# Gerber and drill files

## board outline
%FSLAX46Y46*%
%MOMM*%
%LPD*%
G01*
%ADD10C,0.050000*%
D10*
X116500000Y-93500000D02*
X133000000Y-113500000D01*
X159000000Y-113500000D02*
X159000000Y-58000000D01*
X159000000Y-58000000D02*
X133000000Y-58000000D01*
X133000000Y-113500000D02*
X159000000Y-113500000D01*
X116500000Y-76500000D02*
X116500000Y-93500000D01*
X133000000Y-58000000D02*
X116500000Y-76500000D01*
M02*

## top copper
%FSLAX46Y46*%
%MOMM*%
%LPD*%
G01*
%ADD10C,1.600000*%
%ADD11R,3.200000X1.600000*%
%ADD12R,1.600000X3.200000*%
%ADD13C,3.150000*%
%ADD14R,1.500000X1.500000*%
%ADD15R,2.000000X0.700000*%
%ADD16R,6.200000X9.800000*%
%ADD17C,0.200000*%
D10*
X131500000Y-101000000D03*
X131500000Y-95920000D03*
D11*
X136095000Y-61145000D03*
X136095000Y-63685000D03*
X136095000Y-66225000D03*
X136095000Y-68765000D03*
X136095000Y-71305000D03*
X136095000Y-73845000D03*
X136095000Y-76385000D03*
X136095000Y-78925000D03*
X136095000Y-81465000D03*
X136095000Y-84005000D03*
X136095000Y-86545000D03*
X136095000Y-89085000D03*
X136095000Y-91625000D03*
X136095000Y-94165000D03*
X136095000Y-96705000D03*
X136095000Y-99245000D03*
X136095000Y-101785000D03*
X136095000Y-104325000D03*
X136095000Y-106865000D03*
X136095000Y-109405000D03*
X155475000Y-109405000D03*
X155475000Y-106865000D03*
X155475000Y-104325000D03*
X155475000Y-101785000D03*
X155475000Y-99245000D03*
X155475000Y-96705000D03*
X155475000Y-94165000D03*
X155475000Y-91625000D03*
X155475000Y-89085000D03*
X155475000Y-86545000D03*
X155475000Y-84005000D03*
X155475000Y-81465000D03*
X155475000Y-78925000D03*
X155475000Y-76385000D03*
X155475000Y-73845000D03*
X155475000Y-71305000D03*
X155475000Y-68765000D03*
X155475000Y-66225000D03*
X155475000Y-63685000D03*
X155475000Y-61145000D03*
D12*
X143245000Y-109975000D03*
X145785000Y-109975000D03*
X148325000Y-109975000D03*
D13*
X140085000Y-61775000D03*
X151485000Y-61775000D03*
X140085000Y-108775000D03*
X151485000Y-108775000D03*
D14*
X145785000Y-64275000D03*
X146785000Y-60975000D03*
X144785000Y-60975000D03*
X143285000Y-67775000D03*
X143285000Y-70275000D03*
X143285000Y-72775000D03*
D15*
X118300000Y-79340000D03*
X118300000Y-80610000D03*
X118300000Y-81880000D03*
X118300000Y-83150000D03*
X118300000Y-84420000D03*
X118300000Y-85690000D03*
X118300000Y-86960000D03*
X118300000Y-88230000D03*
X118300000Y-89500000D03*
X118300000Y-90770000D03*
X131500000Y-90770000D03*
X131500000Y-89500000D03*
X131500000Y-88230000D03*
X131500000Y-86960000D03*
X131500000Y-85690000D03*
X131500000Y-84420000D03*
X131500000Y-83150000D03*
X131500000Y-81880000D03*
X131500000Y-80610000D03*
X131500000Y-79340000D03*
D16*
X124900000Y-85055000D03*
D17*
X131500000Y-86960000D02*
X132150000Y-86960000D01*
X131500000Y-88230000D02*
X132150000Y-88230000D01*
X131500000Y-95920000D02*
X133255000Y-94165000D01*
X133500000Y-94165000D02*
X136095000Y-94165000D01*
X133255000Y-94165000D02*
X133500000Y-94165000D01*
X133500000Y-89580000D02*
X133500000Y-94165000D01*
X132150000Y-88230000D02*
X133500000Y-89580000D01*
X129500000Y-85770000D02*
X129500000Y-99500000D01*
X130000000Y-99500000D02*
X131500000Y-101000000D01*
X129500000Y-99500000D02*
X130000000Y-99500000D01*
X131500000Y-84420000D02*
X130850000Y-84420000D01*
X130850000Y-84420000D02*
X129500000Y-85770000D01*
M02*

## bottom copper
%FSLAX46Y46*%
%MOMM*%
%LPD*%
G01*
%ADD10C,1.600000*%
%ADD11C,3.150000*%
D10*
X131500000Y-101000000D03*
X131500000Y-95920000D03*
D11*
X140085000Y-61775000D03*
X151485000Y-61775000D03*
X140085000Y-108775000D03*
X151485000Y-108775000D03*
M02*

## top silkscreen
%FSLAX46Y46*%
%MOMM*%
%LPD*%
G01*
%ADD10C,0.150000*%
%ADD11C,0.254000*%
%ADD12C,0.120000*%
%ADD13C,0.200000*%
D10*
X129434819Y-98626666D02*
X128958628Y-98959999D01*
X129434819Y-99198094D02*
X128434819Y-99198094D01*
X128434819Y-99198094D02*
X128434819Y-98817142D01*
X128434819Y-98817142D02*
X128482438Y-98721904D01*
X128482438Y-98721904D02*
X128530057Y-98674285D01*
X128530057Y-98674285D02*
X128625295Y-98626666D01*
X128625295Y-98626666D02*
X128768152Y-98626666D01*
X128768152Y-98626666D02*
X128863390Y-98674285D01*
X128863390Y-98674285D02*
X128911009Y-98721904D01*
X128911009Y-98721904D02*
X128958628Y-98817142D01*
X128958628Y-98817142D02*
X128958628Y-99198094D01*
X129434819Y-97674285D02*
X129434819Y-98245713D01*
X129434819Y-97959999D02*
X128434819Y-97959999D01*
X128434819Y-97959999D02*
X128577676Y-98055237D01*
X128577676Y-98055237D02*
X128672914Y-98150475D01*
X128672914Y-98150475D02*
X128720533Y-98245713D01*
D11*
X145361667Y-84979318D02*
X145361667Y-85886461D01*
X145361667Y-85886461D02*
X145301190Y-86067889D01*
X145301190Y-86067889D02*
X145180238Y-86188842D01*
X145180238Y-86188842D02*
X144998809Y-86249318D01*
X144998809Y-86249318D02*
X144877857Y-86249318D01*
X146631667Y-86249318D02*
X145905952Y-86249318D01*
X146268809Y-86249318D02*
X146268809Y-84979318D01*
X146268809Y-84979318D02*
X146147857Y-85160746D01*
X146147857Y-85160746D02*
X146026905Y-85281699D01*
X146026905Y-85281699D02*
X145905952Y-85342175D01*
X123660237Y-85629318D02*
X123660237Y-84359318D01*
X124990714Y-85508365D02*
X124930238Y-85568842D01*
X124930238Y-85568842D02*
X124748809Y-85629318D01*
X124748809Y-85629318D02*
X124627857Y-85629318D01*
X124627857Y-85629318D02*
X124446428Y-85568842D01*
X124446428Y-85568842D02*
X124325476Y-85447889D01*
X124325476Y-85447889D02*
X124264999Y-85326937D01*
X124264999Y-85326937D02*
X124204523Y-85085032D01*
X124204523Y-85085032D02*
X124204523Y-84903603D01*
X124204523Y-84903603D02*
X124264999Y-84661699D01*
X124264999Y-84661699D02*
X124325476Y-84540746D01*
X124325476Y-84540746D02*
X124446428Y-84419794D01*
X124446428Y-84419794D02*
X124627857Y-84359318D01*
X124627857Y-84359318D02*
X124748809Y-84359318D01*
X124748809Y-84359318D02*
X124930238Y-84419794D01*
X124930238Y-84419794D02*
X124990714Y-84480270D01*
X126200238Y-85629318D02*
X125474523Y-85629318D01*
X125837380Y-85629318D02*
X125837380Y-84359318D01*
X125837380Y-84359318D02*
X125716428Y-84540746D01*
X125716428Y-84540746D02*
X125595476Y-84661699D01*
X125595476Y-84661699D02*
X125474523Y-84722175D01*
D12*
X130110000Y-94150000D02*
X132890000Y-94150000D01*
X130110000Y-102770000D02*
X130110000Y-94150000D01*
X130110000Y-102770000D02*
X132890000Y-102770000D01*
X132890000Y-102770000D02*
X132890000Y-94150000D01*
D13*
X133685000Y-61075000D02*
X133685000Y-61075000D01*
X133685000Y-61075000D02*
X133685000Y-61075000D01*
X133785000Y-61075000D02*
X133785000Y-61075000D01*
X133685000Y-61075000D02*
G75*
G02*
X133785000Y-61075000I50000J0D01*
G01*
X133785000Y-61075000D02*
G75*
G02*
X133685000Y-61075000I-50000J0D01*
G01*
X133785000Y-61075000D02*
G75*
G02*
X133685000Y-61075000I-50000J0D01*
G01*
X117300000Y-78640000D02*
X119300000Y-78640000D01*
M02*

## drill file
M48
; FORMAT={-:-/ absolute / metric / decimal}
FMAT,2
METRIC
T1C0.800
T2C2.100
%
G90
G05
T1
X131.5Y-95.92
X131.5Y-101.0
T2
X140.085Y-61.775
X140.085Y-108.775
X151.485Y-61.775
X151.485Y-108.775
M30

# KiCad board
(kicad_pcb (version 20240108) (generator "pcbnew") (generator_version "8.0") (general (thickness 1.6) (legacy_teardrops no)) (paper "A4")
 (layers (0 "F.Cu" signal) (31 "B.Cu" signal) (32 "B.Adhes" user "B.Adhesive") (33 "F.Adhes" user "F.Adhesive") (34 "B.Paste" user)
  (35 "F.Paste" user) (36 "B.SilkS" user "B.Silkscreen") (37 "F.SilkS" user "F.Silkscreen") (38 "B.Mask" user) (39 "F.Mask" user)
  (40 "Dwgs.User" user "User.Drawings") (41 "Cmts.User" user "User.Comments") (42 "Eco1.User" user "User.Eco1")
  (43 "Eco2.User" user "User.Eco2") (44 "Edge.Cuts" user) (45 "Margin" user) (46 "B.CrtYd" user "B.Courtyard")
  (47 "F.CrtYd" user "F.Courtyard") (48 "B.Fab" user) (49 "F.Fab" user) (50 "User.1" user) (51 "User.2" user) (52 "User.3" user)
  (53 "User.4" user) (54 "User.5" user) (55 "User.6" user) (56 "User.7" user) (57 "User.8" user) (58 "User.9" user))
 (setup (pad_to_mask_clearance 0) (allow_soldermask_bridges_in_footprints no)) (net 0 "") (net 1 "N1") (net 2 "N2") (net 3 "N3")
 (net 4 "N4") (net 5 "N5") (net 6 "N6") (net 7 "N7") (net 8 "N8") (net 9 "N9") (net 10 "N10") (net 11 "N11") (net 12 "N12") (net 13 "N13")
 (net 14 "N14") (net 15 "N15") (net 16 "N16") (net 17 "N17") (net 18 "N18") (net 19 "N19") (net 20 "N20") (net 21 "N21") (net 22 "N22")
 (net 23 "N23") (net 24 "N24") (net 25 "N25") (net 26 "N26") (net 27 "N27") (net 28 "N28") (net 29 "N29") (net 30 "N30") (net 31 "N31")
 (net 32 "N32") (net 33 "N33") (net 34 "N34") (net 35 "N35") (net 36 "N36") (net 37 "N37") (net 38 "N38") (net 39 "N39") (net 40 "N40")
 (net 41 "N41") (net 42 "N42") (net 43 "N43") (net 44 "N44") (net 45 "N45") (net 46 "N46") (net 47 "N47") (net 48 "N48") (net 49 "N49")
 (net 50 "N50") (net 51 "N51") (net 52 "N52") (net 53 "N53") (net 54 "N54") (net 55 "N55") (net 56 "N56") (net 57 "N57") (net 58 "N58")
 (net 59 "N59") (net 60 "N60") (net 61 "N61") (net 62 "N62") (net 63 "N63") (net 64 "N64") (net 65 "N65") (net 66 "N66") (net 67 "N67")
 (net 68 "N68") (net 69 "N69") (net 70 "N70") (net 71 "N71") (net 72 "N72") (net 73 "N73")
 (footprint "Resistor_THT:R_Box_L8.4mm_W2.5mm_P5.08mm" (layer "F.Cu") (at 131.5 101 90)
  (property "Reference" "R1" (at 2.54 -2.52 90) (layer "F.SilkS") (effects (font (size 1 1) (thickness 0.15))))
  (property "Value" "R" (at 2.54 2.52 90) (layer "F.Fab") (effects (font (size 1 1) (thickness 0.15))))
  (fp_line (start 6.85 -1.39) (end 6.85 1.39) (stroke (width 0.12) (type solid)) (layer "F.SilkS"))
  (fp_line (start -1.77 -1.39) (end 6.85 -1.39) (stroke (width 0.12) (type solid)) (layer "F.SilkS"))
  (fp_line (start -1.77 -1.39) (end -1.77 1.39) (stroke (width 0.12) (type solid)) (layer "F.SilkS"))
  (fp_line (start -1.77 1.39) (end 6.85 1.39) (stroke (width 0.12) (type solid)) (layer "F.SilkS"))
  (pad "1" thru_hole circle (at 0 0 90) (size 1.6 1.6) (drill 0.8) (layers "*.Cu" "*.Mask") (remove_unused_layers no) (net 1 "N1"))
  (pad "2" thru_hole circle (at 5.08 0 90) (size 1.6 1.6) (drill 0.8) (layers "*.Cu" "*.Mask") (remove_unused_layers no) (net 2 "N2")))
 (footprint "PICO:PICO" (layer "F.Cu") (at 145.785 85.275)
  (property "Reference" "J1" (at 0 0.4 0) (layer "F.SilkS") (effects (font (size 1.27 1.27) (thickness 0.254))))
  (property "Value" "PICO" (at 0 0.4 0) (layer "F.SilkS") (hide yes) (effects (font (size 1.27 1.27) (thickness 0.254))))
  (fp_line (start -12.1 -24.2) (end -12.1 -24.2) (stroke (width 0.2) (type solid)) (layer "F.SilkS"))
  (fp_line (start -12.1 -24.2) (end -12.1 -24.2) (stroke (width 0.2) (type solid)) (layer "F.SilkS"))
  (fp_line (start -12 -24.2) (end -12 -24.2) (stroke (width 0.2) (type solid)) (layer "F.SilkS"))
  (fp_arc (start -12.1 -24.2) (mid -12.05 -24.25) (end -12 -24.2) (stroke (width 0.2) (type solid)) (layer "F.SilkS"))
  (fp_arc (start -12 -24.2) (mid -12.05 -24.15) (end -12.1 -24.2) (stroke (width 0.2) (type solid)) (layer "F.SilkS"))
  (fp_arc (start -12 -24.2) (mid -12.05 -24.15) (end -12.1 -24.2) (stroke (width 0.2) (type solid)) (layer "F.SilkS"))
  (pad "1" smd rect (at -9.69 -24.13 90) (size 1.6 3.2) (layers "F.Cu" "F.Paste" "F.Mask") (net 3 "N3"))
  (pad "2" smd rect (at -9.69 -21.59 90) (size 1.6 3.2) (layers "F.Cu" "F.Paste" "F.Mask") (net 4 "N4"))
  (pad "3" smd rect (at -9.69 -19.05 90) (size 1.6 3.2) (layers "F.Cu" "F.Paste" "F.Mask") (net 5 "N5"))
  (pad "4" smd rect (at -9.69 -16.51 90) (size 1.6 3.2) (layers "F.Cu" "F.Paste" "F.Mask") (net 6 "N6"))
  (pad "5" smd rect (at -9.69 -13.97 90) (size 1.6 3.2) (layers "F.Cu" "F.Paste" "F.Mask") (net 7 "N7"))
  (pad "6" smd rect (at -9.69 -11.43 90) (size 1.6 3.2) (layers "F.Cu" "F.Paste" "F.Mask") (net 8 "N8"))
  (pad "7" smd rect (at -9.69 -8.89 90) (size 1.6 3.2) (layers "F.Cu" "F.Paste" "F.Mask") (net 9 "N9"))
  (pad "8" smd rect (at -9.69 -6.35 90) (size 1.6 3.2) (layers "F.Cu" "F.Paste" "F.Mask") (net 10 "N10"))
  (pad "9" smd rect (at -9.69 -3.81 90) (size 1.6 3.2) (layers "F.Cu" "F.Paste" "F.Mask") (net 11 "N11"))
  (pad "10" smd rect (at -9.69 -1.27 90) (size 1.6 3.2) (layers "F.Cu" "F.Paste" "F.Mask") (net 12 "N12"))
  (pad "11" smd rect (at -9.69 1.27 90) (size 1.6 3.2) (layers "F.Cu" "F.Paste" "F.Mask") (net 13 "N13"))
  (pad "12" smd rect (at -9.69 3.81 90) (size 1.6 3.2) (layers "F.Cu" "F.Paste" "F.Mask") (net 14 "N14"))
  (pad "13" smd rect (at -9.69 6.35 90) (size 1.6 3.2) (layers "F.Cu" "F.Paste" "F.Mask") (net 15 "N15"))
  (pad "14" smd rect (at -9.69 8.89 90) (size 1.6 3.2) (layers "F.Cu" "F.Paste" "F.Mask") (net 2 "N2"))
  (pad "15" smd rect (at -9.69 11.43 90) (size 1.6 3.2) (layers "F.Cu" "F.Paste" "F.Mask") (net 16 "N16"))
  (pad "16" smd rect (at -9.69 13.97 90) (size 1.6 3.2) (layers "F.Cu" "F.Paste" "F.Mask") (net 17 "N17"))
  (pad "17" smd rect (at -9.69 16.51 90) (size 1.6 3.2) (layers "F.Cu" "F.Paste" "F.Mask") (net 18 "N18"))
  (pad "18" smd rect (at -9.69 19.05 90) (size 1.6 3.2) (layers "F.Cu" "F.Paste" "F.Mask") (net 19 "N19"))
  (pad "19" smd rect (at -9.69 21.59 90) (size 1.6 3.2) (layers "F.Cu" "F.Paste" "F.Mask") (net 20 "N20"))
  (pad "20" smd rect (at -9.69 24.13 90) (size 1.6 3.2) (layers "F.Cu" "F.Paste" "F.Mask") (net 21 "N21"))
  (pad "21" smd rect (at 9.69 24.13 90) (size 1.6 3.2) (layers "F.Cu" "F.Paste" "F.Mask") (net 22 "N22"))
  (pad "22" smd rect (at 9.69 21.59 90) (size 1.6 3.2) (layers "F.Cu" "F.Paste" "F.Mask") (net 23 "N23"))
  (pad "23" smd rect (at 9.69 19.05 90) (size 1.6 3.2) (layers "F.Cu" "F.Paste" "F.Mask") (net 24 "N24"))
  (pad "24" smd rect (at 9.69 16.51 90) (size 1.6 3.2) (layers "F.Cu" "F.Paste" "F.Mask") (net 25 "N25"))
  (pad "25" smd rect (at 9.69 13.97 90) (size 1.6 3.2) (layers "F.Cu" "F.Paste" "F.Mask") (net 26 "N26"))
  (pad "26" smd rect (at 9.69 11.43 90) (size 1.6 3.2) (layers "F.Cu" "F.Paste" "F.Mask") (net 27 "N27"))
  (pad "27" smd rect (at 9.69 8.89 90) (size 1.6 3.2) (layers "F.Cu" "F.Paste" "F.Mask") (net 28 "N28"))
  (pad "28" smd rect (at 9.69 6.35 90) (size 1.6 3.2) (layers "F.Cu" "F.Paste" "F.Mask") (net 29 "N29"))
  (pad "29" smd rect (at 9.69 3.81 90) (size 1.6 3.2) (layers "F.Cu" "F.Paste" "F.Mask") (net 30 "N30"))
  (pad "30" smd rect (at 9.69 1.27 90) (size 1.6 3.2) (layers "F.Cu" "F.Paste" "F.Mask") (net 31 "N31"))
  (pad "31" smd rect (at 9.69 -1.27 90) (size 1.6 3.2) (layers "F.Cu" "F.Paste" "F.Mask") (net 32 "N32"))
  (pad "32" smd rect (at 9.69 -3.81 90) (size 1.6 3.2) (layers "F.Cu" "F.Paste" "F.Mask") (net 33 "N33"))
  (pad "33" smd rect (at 9.69 -6.35 90) (size 1.6 3.2) (layers "F.Cu" "F.Paste" "F.Mask") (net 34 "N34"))
  (pad "34" smd rect (at 9.69 -8.89 90) (size 1.6 3.2) (layers "F.Cu" "F.Paste" "F.Mask") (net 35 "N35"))
  (pad "35" smd rect (at 9.69 -11.43 90) (size 1.6 3.2) (layers "F.Cu" "F.Paste" "F.Mask") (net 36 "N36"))
  (pad "36" smd rect (at 9.69 -13.97 90) (size 1.6 3.2) (layers "F.Cu" "F.Paste" "F.Mask") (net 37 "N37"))
  (pad "37" smd rect (at 9.69 -16.51 90) (size 1.6 3.2) (layers "F.Cu" "F.Paste" "F.Mask") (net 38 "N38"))
  (pad "38" smd rect (at 9.69 -19.05 90) (size 1.6 3.2) (layers "F.Cu" "F.Paste" "F.Mask") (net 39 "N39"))
  (pad "39" smd rect (at 9.69 -21.59 90) (size 1.6 3.2) (layers "F.Cu" "F.Paste" "F.Mask") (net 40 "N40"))
  (pad "40" smd rect (at 9.69 -24.13 90) (size 1.6 3.2) (layers "F.Cu" "F.Paste" "F.Mask") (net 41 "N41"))
  (pad "D1" smd rect (at -2.54 24.7) (size 1.6 3.2) (layers "F.Cu" "F.Paste" "F.Mask") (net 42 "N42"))
  (pad "D2" smd rect (at 0 24.7) (size 1.6 3.2) (layers "F.Cu" "F.Paste" "F.Mask") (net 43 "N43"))
  (pad "D3" smd rect (at 2.54 24.7) (size 1.6 3.2) (layers "F.Cu" "F.Paste" "F.Mask") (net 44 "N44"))
  (pad "MH1" thru_hole circle (at -5.7 -23.5) (size 3.15 3.15) (drill 2.1) (layers "*.Cu" "*.Mask") (remove_unused_layers no) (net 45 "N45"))
  (pad "MH2" thru_hole circle (at 5.7 -23.5) (size 3.15 3.15) (drill 2.1) (layers "*.Cu" "*.Mask") (remove_unused_layers no) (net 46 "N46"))
  (pad "MH3" thru_hole circle (at -5.7 23.5) (size 3.15 3.15) (drill 2.1) (layers "*.Cu" "*.Mask") (remove_unused_layers no) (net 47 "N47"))
  (pad "MH4" thru_hole circle (at 5.7 23.5) (size 3.15 3.15) (drill 2.1) (layers "*.Cu" "*.Mask") (remove_unused_layers no) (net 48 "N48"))
  (pad "TP1" smd rect (at 0 -21 90) (size 1.5 1.5) (layers "F.Cu" "F.Paste" "F.Mask") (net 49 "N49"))
  (pad "TP2" smd rect (at 1 -24.3 90) (size 1.5 1.5) (layers "F.Cu" "F.Paste" "F.Mask") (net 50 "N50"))
  (pad "TP3" smd rect (at -1 -24.3 90) (size 1.5 1.5) (layers "F.Cu" "F.Paste" "F.Mask") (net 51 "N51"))
  (pad "TP4" smd rect (at -2.5 -17.5 90) (size 1.5 1.5) (layers "F.Cu" "F.Paste" "F.Mask") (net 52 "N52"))
  (pad "TP5" smd rect (at -2.5 -15 90) (size 1.5 1.5) (layers "F.Cu" "F.Paste" "F.Mask") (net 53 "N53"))
  (pad "TP6" smd rect (at -2.5 -12.5 90) (size 1.5 1.5) (layers "F.Cu" "F.Paste" "F.Mask") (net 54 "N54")))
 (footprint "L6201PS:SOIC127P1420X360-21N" (layer "F.Cu") (at 124.9 85.055)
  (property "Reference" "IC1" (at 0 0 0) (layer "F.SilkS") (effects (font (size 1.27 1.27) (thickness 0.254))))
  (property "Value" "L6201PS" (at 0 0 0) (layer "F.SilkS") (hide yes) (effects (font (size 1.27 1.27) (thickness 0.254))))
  (fp_line (start -7.6 -6.415) (end -5.6 -6.415) (stroke (width 0.2) (type solid)) (layer "F.SilkS"))
  (pad "1" smd rect (at -6.6 -5.715 90) (size 0.7 2) (layers "F.Cu" "F.Paste" "F.Mask") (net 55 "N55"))
  (pad "2" smd rect (at -6.6 -4.445 90) (size 0.7 2) (layers "F.Cu" "F.Paste" "F.Mask") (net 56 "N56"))
  (pad "3" smd rect (at -6.6 -3.175 90) (size 0.7 2) (layers "F.Cu" "F.Paste" "F.Mask") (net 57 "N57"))
  (pad "4" smd rect (at -6.6 -1.905 90) (size 0.7 2) (layers "F.Cu" "F.Paste" "F.Mask") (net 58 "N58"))
  (pad "5" smd rect (at -6.6 -0.635 90) (size 0.7 2) (layers "F.Cu" "F.Paste" "F.Mask") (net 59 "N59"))
  (pad "6" smd rect (at -6.6 0.635 90) (size 0.7 2) (layers "F.Cu" "F.Paste" "F.Mask") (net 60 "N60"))
  (pad "7" smd rect (at -6.6 1.905 90) (size 0.7 2) (layers "F.Cu" "F.Paste" "F.Mask") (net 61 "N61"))
  (pad "8" smd rect (at -6.6 3.175 90) (size 0.7 2) (layers "F.Cu" "F.Paste" "F.Mask") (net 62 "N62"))
  (pad "9" smd rect (at -6.6 4.445 90) (size 0.7 2) (layers "F.Cu" "F.Paste" "F.Mask") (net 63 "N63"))
  (pad "10" smd rect (at -6.6 5.715 90) (size 0.7 2) (layers "F.Cu" "F.Paste" "F.Mask") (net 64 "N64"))
  (pad "11" smd rect (at 6.6 5.715 90) (size 0.7 2) (layers "F.Cu" "F.Paste" "F.Mask") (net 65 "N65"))
  (pad "12" smd rect (at 6.6 4.445 90) (size 0.7 2) (layers "F.Cu" "F.Paste" "F.Mask") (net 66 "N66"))
  (pad "13" smd rect (at 6.6 3.175 90) (size 0.7 2) (layers "F.Cu" "F.Paste" "F.Mask") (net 2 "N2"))
  (pad "14" smd rect (at 6.6 1.905 90) (size 0.7 2) (layers "F.Cu" "F.Paste" "F.Mask") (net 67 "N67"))
  (pad "15" smd rect (at 6.6 0.635 90) (size 0.7 2) (layers "F.Cu" "F.Paste" "F.Mask") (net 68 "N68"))
  (pad "16" smd rect (at 6.6 -0.635 90) (size 0.7 2) (layers "F.Cu" "F.Paste" "F.Mask") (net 1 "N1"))
  (pad "17" smd rect (at 6.6 -1.905 90) (size 0.7 2) (layers "F.Cu" "F.Paste" "F.Mask") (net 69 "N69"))
  (pad "18" smd rect (at 6.6 -3.175 90) (size 0.7 2) (layers "F.Cu" "F.Paste" "F.Mask") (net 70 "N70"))
  (pad "19" smd rect (at 6.6 -4.445 90) (size 0.7 2) (layers "F.Cu" "F.Paste" "F.Mask") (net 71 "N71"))
  (pad "20" smd rect (at 6.6 -5.715 90) (size 0.7 2) (layers "F.Cu" "F.Paste" "F.Mask") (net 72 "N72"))
  (pad "21" smd rect (at 0 0) (size 6.2 9.8) (layers "F.Cu" "F.Paste" "F.Mask") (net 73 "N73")))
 (gr_line (start 116.5 93.5) (end 133 113.5) (stroke (width 0.05) (type default)) (layer "Edge.Cuts"))
 (gr_line (start 159 113.5) (end 159 58) (stroke (width 0.05) (type default)) (layer "Edge.Cuts"))
 (gr_line (start 159 58) (end 133 58) (stroke (width 0.05) (type default)) (layer "Edge.Cuts"))
 (gr_line (start 133 113.5) (end 159 113.5) (stroke (width 0.05) (type default)) (layer "Edge.Cuts"))
 (gr_line (start 116.5 76.5) (end 116.5 93.5) (stroke (width 0.05) (type default)) (layer "Edge.Cuts"))
 (gr_line (start 133 58) (end 116.5 76.5) (stroke (width 0.05) (type default)) (layer "Edge.Cuts"))
 (segment (start 131.5 86.96) (end 132.15 86.96) (width 0.2) (layer "F.Cu") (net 67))
 (segment (start 131.5 88.23) (end 132.15 88.23) (width 0.2) (layer "F.Cu") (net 2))
 (segment (start 131.5 95.92) (end 133.255 94.165) (width 0.2) (layer "F.Cu") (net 2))
 (segment (start 133.5 94.165) (end 136.095 94.165) (width 0.2) (layer "F.Cu") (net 2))
 (segment (start 133.255 94.165) (end 133.5 94.165) (width 0.2) (layer "F.Cu") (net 2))
 (segment (start 133.5 89.58) (end 133.5 94.165) (width 0.2) (layer "F.Cu") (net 2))
 (segment (start 132.15 88.23) (end 133.5 89.58) (width 0.2) (layer "F.Cu") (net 2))
 (segment (start 129.5 85.77) (end 129.5 99.5) (width 0.2) (layer "F.Cu") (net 1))
 (segment (start 130 99.5) (end 131.5 101) (width 0.2) (layer "F.Cu") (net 1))
 (segment (start 129.5 99.5) (end 130 99.5) (width 0.2) (layer "F.Cu") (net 1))
 (segment (start 131.5 84.42) (end 130.85 84.42) (width 0.2) (layer "F.Cu") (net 1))
 (segment (start 130.85 84.42) (end 129.5 85.77) (width 0.2) (layer "F.Cu") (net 1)))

